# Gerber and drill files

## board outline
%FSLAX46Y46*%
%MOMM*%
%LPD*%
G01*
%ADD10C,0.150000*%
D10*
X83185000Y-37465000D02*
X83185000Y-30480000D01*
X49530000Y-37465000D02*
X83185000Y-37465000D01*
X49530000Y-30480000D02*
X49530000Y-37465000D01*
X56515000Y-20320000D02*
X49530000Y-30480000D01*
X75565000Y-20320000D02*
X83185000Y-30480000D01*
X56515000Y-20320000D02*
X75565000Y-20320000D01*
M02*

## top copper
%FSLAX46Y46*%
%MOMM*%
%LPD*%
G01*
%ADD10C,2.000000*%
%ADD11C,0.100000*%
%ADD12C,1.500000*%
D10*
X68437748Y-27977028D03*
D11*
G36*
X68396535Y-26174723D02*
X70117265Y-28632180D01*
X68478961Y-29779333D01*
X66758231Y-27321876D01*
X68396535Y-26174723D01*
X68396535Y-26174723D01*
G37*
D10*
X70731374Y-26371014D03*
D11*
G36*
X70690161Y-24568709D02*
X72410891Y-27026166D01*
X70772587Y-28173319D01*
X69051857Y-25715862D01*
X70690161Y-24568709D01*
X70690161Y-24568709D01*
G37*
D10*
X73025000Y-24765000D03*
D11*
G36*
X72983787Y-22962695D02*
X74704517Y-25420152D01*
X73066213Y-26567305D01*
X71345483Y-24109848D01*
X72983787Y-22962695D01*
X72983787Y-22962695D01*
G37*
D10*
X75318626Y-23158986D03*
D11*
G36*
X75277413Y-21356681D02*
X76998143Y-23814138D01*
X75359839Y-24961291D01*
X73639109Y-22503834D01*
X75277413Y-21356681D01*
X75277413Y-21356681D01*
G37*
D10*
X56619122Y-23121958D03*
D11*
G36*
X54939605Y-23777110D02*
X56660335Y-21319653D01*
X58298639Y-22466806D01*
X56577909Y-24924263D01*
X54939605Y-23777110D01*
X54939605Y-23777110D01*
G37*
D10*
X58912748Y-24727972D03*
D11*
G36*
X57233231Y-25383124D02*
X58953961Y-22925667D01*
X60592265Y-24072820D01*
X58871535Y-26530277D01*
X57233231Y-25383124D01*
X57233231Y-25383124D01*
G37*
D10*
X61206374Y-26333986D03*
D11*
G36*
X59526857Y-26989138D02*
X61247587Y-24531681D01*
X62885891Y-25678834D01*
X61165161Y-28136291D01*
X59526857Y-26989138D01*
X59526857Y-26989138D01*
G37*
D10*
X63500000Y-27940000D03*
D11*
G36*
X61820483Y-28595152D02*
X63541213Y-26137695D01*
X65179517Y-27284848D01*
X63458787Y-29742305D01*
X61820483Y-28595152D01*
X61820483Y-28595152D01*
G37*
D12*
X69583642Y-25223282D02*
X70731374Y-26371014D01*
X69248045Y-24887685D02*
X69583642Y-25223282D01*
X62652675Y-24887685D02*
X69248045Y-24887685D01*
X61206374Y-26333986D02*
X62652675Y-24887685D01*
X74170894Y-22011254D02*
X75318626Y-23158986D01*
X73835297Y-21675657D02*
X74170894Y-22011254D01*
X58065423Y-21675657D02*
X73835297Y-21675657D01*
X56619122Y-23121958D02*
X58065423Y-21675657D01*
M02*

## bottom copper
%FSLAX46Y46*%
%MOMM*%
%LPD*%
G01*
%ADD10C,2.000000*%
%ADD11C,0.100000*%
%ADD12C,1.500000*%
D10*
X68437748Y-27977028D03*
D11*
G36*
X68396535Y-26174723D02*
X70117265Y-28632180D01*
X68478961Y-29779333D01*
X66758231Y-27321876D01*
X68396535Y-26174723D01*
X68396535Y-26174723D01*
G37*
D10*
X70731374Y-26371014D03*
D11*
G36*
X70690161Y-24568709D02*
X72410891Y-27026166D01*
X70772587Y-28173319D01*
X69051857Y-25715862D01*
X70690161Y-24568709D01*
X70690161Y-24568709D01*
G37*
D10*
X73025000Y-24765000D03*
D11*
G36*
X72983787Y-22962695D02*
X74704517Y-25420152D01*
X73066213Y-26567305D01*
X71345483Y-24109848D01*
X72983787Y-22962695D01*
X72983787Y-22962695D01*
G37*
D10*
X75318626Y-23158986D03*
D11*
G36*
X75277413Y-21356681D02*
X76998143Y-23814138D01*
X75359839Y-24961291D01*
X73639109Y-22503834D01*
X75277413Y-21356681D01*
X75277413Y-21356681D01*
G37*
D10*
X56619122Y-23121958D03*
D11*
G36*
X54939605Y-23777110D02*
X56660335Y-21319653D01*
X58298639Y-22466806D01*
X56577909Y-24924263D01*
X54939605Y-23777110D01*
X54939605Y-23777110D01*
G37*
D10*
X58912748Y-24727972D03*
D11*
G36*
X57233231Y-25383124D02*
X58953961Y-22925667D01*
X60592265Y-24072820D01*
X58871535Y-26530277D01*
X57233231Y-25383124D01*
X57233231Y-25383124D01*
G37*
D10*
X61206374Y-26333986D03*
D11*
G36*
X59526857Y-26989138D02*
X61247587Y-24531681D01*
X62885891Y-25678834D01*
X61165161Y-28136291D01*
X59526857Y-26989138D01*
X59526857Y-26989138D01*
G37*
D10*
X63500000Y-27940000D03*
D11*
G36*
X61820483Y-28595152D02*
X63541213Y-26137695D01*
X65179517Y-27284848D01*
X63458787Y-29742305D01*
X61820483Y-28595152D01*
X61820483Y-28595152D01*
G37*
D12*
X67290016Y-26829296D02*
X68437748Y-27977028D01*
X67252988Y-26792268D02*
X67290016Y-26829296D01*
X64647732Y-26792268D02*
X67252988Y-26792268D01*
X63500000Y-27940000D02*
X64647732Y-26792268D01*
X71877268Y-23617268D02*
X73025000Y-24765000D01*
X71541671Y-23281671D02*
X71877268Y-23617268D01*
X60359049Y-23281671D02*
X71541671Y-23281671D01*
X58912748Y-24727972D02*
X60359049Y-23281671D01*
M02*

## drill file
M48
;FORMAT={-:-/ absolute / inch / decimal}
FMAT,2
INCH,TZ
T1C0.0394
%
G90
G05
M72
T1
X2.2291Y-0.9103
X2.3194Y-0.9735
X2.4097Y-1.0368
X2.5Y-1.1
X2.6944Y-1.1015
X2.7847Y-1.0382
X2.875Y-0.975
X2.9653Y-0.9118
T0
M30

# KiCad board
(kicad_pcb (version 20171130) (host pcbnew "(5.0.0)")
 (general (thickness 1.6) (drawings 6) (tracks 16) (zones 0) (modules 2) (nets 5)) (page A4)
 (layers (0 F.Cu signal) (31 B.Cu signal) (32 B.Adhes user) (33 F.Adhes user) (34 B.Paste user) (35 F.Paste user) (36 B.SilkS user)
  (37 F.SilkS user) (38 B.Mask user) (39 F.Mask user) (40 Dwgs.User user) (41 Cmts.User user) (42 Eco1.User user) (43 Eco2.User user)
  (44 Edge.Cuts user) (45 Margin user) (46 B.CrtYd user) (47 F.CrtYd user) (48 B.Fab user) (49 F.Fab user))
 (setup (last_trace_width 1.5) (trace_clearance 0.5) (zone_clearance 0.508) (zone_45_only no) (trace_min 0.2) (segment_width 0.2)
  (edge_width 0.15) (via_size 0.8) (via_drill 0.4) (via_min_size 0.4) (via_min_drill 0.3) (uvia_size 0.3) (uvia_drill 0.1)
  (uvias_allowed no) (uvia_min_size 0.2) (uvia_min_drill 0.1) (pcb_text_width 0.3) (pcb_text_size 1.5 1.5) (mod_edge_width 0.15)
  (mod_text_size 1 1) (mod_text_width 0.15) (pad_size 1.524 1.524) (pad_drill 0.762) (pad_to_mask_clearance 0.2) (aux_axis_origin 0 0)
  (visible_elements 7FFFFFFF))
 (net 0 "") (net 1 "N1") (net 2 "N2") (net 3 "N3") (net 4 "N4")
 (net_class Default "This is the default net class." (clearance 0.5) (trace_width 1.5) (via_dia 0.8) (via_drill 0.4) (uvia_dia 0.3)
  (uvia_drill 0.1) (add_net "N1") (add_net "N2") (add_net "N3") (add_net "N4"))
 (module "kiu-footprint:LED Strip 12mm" (layer F.Cu) (at 71.878187 25.568007 215)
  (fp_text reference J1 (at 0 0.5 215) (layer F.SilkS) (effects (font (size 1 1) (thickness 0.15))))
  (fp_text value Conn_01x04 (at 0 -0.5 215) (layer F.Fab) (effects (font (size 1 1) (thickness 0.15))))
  (pad 1 thru_hole rect (at 4.2 0 215) (size 2 3) (drill 1) (layers *.Cu *.Mask) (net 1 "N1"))
  (pad 2 thru_hole rect (at 1.4 0 215) (size 2 3) (drill 1) (layers *.Cu *.Mask) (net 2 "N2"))
  (pad 3 thru_hole rect (at -1.4 0 215) (size 2 3) (drill 1) (layers *.Cu *.Mask) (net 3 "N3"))
  (pad 4 thru_hole rect (at -4.2 0 215) (size 2 3) (drill 1) (layers *.Cu *.Mask) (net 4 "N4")))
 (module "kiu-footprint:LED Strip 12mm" (layer F.Cu) (at 60.059561 25.530979 325)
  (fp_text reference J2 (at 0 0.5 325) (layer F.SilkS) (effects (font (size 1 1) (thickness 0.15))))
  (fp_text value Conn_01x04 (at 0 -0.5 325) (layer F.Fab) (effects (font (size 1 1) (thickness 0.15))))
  (pad 4 thru_hole rect (at -4.2 0 325) (size 2 3) (drill 1) (layers *.Cu *.Mask) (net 4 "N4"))
  (pad 3 thru_hole rect (at -1.4 0 325) (size 2 3) (drill 1) (layers *.Cu *.Mask) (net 3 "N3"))
  (pad 2 thru_hole rect (at 1.4 0 325) (size 2 3) (drill 1) (layers *.Cu *.Mask) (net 2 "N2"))
  (pad 1 thru_hole rect (at 4.2 0 325) (size 2 3) (drill 1) (layers *.Cu *.Mask) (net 1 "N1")))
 (gr_line (start 83.185 37.465) (end 83.185 30.48) (layer Edge.Cuts) (width 0.15))
 (gr_line (start 49.53 37.465) (end 83.185 37.465) (layer Edge.Cuts) (width 0.15))
 (gr_line (start 49.53 30.48) (end 49.53 37.465) (layer Edge.Cuts) (width 0.15))
 (gr_line (start 56.515 20.32) (end 49.53 30.48) (layer Edge.Cuts) (width 0.15))
 (gr_line (start 75.565 20.32) (end 83.185 30.48) (layer Edge.Cuts) (width 0.15))
 (gr_line (start 56.515 20.32) (end 75.565 20.32) (layer Edge.Cuts) (width 0.15))
 (segment (start 67.290016 26.829296) (end 68.437748 27.977028) (width 1.5) (layer B.Cu) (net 1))
 (segment (start 67.252988 26.792268) (end 67.290016 26.829296) (width 1.5) (layer B.Cu) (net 1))
 (segment (start 64.647732 26.792268) (end 67.252988 26.792268) (width 1.5) (layer B.Cu) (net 1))
 (segment (start 63.5 27.94) (end 64.647732 26.792268) (width 1.5) (layer B.Cu) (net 1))
 (segment (start 69.583642 25.223282) (end 70.731374 26.371014) (width 1.5) (layer F.Cu) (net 2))
 (segment (start 69.248045 24.887685) (end 69.583642 25.223282) (width 1.5) (layer F.Cu) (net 2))
 (segment (start 62.652675 24.887685) (end 69.248045 24.887685) (width 1.5) (layer F.Cu) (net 2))
 (segment (start 61.206374 26.333986) (end 62.652675 24.887685) (width 1.5) (layer F.Cu) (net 2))
 (segment (start 71.877268 23.617268) (end 73.025 24.765) (width 1.5) (layer B.Cu) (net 3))
 (segment (start 71.541671 23.281671) (end 71.877268 23.617268) (width 1.5) (layer B.Cu) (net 3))
 (segment (start 60.359049 23.281671) (end 71.541671 23.281671) (width 1.5) (layer B.Cu) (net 3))
 (segment (start 58.912748 24.727972) (end 60.359049 23.281671) (width 1.5) (layer B.Cu) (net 3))
 (segment (start 74.170894 22.011254) (end 75.318626 23.158986) (width 1.5) (layer F.Cu) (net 4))
 (segment (start 73.835297 21.675657) (end 74.170894 22.011254) (width 1.5) (layer F.Cu) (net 4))
 (segment (start 58.065423 21.675657) (end 73.835297 21.675657) (width 1.5) (layer F.Cu) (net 4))
 (segment (start 56.619122 23.121958) (end 58.065423 21.675657) (width 1.5) (layer F.Cu) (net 4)))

